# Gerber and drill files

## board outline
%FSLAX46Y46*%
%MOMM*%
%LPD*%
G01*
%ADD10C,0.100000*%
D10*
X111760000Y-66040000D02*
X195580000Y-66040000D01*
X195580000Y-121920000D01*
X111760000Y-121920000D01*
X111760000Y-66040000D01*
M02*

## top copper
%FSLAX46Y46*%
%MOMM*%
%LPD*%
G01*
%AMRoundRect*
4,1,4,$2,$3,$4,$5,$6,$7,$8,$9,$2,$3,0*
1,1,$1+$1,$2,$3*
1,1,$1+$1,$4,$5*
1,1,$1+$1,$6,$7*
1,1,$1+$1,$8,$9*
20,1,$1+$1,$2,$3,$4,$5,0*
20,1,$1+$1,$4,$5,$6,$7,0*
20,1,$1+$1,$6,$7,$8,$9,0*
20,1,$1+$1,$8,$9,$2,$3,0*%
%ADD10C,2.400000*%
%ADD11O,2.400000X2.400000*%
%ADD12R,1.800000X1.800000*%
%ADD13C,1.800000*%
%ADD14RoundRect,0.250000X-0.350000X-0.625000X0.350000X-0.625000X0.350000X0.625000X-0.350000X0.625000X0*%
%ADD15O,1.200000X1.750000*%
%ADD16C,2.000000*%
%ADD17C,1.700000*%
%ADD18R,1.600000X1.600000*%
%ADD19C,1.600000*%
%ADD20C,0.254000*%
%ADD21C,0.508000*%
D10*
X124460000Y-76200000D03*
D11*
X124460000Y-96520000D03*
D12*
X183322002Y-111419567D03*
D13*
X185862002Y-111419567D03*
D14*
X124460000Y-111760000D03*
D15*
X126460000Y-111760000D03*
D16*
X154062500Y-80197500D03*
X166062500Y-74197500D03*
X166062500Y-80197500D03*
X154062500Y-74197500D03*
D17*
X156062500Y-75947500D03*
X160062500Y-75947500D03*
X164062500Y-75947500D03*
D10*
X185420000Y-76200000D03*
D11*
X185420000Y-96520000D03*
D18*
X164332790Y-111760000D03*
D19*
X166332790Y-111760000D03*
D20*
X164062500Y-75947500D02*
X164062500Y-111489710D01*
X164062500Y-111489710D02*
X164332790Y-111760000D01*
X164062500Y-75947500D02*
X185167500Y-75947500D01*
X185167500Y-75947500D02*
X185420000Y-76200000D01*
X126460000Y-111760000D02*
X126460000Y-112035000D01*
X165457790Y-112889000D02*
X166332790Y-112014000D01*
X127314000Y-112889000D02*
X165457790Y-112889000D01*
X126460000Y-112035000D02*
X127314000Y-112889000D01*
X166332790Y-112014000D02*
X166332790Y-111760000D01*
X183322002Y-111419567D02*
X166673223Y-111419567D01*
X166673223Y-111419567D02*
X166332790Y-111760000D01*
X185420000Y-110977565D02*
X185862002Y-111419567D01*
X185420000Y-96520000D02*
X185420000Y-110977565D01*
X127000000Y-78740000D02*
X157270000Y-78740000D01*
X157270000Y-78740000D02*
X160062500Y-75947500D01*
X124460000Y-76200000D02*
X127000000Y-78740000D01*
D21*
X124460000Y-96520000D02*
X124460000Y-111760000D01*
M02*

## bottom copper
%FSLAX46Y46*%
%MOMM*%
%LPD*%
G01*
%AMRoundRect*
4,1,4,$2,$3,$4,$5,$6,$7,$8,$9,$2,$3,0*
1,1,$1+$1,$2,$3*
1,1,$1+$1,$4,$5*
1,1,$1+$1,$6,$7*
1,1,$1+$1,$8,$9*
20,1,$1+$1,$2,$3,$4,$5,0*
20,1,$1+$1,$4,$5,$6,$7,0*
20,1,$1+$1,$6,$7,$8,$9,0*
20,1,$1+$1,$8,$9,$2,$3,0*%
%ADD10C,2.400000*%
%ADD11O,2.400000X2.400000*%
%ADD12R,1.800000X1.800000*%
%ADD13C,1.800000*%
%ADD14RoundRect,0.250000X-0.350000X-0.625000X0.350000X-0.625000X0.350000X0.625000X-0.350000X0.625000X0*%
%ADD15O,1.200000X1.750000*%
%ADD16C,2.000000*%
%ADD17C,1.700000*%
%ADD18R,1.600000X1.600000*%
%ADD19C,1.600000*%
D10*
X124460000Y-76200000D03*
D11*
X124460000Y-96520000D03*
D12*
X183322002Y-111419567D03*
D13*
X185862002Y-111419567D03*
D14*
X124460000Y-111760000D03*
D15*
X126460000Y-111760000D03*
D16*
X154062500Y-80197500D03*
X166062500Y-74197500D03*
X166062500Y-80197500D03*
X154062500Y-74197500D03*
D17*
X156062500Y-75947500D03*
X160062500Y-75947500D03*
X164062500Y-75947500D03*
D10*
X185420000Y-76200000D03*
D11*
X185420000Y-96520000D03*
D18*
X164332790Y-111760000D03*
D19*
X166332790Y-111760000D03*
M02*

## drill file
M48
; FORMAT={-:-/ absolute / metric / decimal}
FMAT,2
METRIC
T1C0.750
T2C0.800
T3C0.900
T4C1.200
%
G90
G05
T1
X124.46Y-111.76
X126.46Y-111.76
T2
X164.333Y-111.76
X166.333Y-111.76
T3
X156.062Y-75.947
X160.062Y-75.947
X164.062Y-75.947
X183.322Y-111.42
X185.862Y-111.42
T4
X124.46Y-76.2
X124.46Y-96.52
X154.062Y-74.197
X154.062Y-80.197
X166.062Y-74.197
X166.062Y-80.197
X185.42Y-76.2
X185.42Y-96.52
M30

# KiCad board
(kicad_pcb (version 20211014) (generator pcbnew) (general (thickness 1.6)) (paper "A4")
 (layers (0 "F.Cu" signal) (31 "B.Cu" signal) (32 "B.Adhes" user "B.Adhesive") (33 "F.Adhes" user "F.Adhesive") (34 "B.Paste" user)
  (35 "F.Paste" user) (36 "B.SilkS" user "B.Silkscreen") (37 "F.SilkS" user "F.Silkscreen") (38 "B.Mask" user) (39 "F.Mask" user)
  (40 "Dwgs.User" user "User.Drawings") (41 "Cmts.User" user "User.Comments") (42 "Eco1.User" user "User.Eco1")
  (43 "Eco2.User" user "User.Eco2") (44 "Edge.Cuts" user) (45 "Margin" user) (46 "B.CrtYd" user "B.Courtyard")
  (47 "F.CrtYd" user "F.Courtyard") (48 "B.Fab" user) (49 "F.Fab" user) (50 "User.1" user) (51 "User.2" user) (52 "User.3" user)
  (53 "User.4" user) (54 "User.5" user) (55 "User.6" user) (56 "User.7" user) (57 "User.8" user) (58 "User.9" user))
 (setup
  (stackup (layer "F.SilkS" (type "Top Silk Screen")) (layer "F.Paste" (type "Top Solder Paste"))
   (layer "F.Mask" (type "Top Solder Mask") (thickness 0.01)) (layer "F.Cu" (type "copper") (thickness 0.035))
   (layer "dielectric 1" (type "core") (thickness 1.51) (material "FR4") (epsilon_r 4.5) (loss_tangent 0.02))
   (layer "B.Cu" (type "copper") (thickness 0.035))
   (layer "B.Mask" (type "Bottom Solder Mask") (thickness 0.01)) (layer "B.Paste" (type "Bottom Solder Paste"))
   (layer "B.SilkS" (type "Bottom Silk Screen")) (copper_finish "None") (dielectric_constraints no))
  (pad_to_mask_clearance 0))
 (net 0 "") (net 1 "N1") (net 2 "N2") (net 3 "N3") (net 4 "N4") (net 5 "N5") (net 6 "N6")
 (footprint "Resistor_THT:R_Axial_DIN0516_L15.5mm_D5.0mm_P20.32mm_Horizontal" (layer "F.Cu") (at 124.46 76.2 -90)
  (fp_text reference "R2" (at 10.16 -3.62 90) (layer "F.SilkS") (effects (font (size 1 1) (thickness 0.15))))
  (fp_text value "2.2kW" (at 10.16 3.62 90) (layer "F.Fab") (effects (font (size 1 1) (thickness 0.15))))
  (pad "1" thru_hole circle (at 0 0 270) (size 2.4 2.4) (drill 1.2) (layers *.Cu *.Mask) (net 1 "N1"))
  (pad "2" thru_hole oval (at 20.32 0 270) (size 2.4 2.4) (drill 1.2) (layers *.Cu *.Mask) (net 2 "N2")))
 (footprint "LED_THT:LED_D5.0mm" (layer "F.Cu") (at 183.322002 111.419567)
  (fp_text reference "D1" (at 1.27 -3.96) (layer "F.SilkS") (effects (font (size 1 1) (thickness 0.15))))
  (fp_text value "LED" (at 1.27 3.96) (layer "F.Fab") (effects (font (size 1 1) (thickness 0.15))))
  (pad "1" thru_hole rect (at 0 0) (size 1.8 1.8) (drill 0.9) (layers *.Cu *.Mask) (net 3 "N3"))
  (pad "2" thru_hole circle (at 2.54 0) (size 1.8 1.8) (drill 0.9) (layers *.Cu *.Mask) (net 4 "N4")))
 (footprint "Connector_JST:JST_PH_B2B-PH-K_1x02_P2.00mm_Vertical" (layer "F.Cu") (at 124.46 111.76)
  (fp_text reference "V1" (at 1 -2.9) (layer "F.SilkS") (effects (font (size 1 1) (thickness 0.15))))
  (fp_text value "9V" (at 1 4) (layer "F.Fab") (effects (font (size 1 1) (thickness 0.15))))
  (pad "1" thru_hole roundrect (at 0 0) (size 1.2 1.75) (drill 0.75) (layers *.Cu *.Mask) (roundrect_rratio 0.208333) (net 2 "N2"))
  (pad "2" thru_hole oval (at 2 0) (size 1.2 1.75) (drill 0.75) (layers *.Cu *.Mask) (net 3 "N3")))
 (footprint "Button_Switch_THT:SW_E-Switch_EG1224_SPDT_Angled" (layer "F.Cu") (at 156.0625 75.9475)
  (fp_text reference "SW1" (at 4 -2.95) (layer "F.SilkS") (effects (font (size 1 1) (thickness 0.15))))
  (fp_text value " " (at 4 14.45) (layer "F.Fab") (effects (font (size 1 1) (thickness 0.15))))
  (pad "" thru_hole circle (at -2 4.25) (size 2 2) (drill 1.2) (layers *.Cu *.Mask))
  (pad "" thru_hole circle (at 10 -1.75) (size 2 2) (drill 1.2) (layers *.Cu *.Mask))
  (pad "" thru_hole circle (at 10 4.25) (size 2 2) (drill 1.2) (layers *.Cu *.Mask))
  (pad "" thru_hole circle (at -2 -1.75) (size 2 2) (drill 1.2) (layers *.Cu *.Mask))
  (pad "1" thru_hole circle (at 0 0) (size 1.7 1.7) (drill 0.9) (layers *.Cu *.Mask) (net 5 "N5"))
  (pad "2" thru_hole circle (at 4 0) (size 1.7 1.7) (drill 0.9) (layers *.Cu *.Mask) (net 1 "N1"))
  (pad "3" thru_hole circle (at 8 0) (size 1.7 1.7) (drill 0.9) (layers *.Cu *.Mask) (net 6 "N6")))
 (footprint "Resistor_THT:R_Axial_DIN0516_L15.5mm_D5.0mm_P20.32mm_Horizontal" (layer "F.Cu") (at 185.42 76.2 -90)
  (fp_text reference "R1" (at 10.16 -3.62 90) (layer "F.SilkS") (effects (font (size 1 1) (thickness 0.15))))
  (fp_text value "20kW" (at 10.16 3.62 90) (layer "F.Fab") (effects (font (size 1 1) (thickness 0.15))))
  (pad "1" thru_hole circle (at 0 0 270) (size 2.4 2.4) (drill 1.2) (layers *.Cu *.Mask) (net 6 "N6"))
  (pad "2" thru_hole oval (at 20.32 0 270) (size 2.4 2.4) (drill 1.2) (layers *.Cu *.Mask) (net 4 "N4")))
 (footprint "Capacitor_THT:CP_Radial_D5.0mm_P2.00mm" (layer "F.Cu") (at 164.33279 111.76)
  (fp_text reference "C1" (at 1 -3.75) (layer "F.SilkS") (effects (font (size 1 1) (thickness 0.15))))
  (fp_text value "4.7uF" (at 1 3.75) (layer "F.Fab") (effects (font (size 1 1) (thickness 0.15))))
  (pad "1" thru_hole rect (at 0 0) (size 1.6 1.6) (drill 0.8) (layers *.Cu *.Mask) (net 6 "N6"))
  (pad "2" thru_hole circle (at 2 0) (size 1.6 1.6) (drill 0.8) (layers *.Cu *.Mask) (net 3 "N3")))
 (gr_rect (start 111.76 66.04) (end 195.58 121.92) (layer "Edge.Cuts") (width 0.1) (fill none))
 (segment (start 164.0625 75.9475) (end 164.0625 111.48971) (width 0.254) (layer "F.Cu") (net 6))
 (segment (start 164.0625 111.48971) (end 164.33279 111.76) (width 0.254) (layer "F.Cu") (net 6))
 (segment (start 164.0625 75.9475) (end 185.1675 75.9475) (width 0.254) (layer "F.Cu") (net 6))
 (segment (start 185.1675 75.9475) (end 185.42 76.2) (width 0.254) (layer "F.Cu") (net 6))
 (segment (start 126.46 111.76) (end 126.46 112.035) (width 0.254) (layer "F.Cu") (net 3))
 (segment (start 165.45779 112.889) (end 166.33279 112.014) (width 0.254) (layer "F.Cu") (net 3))
 (segment (start 127.314 112.889) (end 165.45779 112.889) (width 0.254) (layer "F.Cu") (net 3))
 (segment (start 126.46 112.035) (end 127.314 112.889) (width 0.254) (layer "F.Cu") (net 3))
 (segment (start 166.33279 112.014) (end 166.33279 111.76) (width 0.254) (layer "F.Cu") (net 3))
 (segment (start 183.322002 111.419567) (end 166.673223 111.419567) (width 0.254) (layer "F.Cu") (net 3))
 (segment (start 166.673223 111.419567) (end 166.33279 111.76) (width 0.254) (layer "F.Cu") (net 3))
 (segment (start 185.42 110.977565) (end 185.862002 111.419567) (width 0.254) (layer "F.Cu") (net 4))
 (segment (start 185.42 96.52) (end 185.42 110.977565) (width 0.254) (layer "F.Cu") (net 4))
 (segment (start 127 78.74) (end 157.27 78.74) (width 0.254) (layer "F.Cu") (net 1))
 (segment (start 157.27 78.74) (end 160.0625 75.9475) (width 0.254) (layer "F.Cu") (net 1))
 (segment (start 124.46 76.2) (end 127 78.74) (width 0.254) (layer "F.Cu") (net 1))
 (segment (start 124.46 96.52) (end 124.46 111.76) (width 0.508) (layer "F.Cu") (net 2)))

